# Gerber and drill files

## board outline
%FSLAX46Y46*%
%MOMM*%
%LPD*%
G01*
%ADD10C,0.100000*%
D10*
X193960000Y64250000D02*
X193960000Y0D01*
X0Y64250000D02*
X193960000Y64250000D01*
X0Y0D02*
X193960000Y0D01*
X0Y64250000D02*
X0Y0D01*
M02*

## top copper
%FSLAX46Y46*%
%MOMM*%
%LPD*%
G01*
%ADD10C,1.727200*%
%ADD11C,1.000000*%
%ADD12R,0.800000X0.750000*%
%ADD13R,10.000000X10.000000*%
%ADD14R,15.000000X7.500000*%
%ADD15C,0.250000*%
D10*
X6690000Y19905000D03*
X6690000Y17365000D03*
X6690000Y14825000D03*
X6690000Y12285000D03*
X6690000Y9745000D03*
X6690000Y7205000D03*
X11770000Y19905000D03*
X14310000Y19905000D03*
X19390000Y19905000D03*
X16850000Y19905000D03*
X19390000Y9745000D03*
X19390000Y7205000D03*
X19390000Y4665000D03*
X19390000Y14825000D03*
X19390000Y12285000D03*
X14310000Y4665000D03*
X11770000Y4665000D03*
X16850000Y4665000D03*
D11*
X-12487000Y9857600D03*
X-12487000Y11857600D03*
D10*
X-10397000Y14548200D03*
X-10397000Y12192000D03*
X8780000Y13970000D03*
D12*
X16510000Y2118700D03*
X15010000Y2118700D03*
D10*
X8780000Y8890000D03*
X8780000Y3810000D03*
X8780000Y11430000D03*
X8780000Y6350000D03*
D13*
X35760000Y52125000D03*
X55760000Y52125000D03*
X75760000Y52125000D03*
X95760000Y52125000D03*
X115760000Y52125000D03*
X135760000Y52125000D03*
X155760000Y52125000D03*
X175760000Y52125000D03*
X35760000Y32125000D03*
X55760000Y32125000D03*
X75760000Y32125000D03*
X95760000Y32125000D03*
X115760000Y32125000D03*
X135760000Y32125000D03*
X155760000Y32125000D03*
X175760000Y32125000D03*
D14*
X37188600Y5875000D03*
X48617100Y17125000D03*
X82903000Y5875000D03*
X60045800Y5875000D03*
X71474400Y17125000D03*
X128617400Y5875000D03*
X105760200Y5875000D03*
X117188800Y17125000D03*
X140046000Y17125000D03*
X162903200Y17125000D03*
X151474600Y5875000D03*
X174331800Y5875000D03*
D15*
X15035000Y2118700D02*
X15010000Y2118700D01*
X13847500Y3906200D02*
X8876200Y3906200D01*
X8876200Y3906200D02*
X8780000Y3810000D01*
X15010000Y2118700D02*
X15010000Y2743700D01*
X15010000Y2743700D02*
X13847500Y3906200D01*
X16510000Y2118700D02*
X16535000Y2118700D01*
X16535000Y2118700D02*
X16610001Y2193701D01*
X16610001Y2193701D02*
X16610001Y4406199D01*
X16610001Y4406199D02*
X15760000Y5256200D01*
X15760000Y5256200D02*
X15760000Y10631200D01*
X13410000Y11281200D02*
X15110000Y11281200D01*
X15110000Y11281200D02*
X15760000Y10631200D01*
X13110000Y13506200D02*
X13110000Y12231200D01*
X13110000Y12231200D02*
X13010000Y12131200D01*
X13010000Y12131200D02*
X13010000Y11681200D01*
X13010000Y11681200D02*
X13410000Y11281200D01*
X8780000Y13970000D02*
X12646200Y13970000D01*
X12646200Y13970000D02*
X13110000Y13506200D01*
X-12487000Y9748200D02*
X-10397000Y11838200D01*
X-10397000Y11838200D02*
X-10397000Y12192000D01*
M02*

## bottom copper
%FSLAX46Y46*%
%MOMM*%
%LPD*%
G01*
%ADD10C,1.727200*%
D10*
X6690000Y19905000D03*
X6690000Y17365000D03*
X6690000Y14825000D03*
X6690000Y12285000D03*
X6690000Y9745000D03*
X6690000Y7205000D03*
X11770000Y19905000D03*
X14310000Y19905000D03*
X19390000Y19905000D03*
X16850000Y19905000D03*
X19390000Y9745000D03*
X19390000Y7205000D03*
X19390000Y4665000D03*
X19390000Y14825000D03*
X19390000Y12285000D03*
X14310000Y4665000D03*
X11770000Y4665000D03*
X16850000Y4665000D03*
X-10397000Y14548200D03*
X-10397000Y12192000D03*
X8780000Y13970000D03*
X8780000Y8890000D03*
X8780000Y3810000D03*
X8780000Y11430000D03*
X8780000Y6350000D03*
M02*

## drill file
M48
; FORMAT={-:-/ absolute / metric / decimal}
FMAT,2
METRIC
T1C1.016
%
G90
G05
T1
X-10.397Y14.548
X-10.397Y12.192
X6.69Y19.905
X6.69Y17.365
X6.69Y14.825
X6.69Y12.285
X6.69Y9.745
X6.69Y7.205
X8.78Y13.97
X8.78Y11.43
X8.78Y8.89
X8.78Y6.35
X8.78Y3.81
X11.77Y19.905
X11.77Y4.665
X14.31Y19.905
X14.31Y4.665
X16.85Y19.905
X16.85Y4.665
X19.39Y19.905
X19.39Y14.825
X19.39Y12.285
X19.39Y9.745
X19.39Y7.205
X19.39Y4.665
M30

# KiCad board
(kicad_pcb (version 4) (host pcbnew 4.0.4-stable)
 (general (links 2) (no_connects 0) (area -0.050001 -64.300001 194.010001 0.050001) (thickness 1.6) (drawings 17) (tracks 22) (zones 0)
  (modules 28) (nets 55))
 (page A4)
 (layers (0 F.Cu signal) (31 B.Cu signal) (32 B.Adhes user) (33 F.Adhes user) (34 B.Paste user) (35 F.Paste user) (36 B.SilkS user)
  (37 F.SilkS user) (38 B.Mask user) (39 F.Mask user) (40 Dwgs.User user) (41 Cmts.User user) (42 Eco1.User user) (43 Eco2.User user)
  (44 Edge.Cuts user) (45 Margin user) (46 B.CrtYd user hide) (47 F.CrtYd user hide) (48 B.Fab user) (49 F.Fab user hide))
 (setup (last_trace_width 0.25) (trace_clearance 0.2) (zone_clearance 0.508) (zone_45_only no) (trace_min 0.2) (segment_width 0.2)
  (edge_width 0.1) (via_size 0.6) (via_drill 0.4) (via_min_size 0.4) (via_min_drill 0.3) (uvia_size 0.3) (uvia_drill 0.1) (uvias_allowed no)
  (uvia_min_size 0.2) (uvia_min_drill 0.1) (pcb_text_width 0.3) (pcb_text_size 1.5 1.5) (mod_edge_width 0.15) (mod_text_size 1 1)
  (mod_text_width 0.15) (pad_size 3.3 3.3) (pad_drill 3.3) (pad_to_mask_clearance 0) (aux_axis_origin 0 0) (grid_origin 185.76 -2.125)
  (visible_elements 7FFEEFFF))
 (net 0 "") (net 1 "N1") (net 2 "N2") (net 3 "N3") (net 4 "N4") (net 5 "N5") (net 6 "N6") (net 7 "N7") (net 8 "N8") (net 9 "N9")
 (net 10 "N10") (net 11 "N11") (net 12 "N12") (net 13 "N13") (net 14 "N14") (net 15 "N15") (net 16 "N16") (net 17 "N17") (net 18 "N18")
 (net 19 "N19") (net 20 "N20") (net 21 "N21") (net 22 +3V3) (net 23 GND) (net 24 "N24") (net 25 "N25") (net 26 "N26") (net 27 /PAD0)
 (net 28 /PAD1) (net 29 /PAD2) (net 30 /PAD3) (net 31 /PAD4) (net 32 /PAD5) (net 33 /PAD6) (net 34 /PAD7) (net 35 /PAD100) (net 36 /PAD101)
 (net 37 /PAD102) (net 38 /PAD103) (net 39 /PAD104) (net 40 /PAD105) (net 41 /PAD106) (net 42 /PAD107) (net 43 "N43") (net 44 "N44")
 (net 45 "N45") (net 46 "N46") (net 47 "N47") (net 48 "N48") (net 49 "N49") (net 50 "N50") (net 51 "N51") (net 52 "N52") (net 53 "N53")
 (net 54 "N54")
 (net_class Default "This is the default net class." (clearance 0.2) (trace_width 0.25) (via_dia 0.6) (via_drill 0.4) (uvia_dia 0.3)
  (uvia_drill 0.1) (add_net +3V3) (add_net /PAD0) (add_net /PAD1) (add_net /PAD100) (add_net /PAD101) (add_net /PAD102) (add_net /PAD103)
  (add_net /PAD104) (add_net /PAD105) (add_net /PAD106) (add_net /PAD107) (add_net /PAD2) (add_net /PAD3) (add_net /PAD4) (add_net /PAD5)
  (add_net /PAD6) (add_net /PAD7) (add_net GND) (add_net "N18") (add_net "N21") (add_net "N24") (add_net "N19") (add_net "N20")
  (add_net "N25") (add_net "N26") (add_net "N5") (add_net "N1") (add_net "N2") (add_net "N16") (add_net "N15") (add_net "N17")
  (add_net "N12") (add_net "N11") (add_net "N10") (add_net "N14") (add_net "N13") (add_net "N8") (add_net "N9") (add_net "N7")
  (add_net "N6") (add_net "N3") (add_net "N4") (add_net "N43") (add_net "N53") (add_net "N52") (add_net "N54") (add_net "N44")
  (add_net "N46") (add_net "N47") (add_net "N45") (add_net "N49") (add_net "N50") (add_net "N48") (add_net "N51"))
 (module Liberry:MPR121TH (layer F.Cu) (at 6.69 -19.905)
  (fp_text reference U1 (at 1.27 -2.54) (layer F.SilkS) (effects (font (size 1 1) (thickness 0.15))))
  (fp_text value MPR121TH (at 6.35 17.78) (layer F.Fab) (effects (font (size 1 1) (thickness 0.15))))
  (pad +3V3 thru_hole circle (at 0 0) (size 1.7272 1.7272) (drill 1.016) (layers *.Cu *.Mask))
  (pad GND thru_hole circle (at 0 2.54) (size 1.7272 1.7272) (drill 1.016) (layers *.Cu *.Mask) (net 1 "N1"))
  (pad IRQ thru_hole circle (at 0 5.08) (size 1.7272 1.7272) (drill 1.016) (layers *.Cu *.Mask) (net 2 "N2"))
  (pad SCL thru_hole circle (at 0 7.62) (size 1.7272 1.7272) (drill 1.016) (layers *.Cu *.Mask) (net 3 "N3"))
  (pad SDA thru_hole circle (at 0 10.16) (size 1.7272 1.7272) (drill 1.016) (layers *.Cu *.Mask) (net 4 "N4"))
  (pad ADDR thru_hole circle (at 0 12.7) (size 1.7272 1.7272) (drill 1.016) (layers *.Cu *.Mask) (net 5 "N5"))
  (pad P11 thru_hole circle (at 5.08 0) (size 1.7272 1.7272) (drill 1.016) (layers *.Cu *.Mask) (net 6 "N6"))
  (pad P10 thru_hole circle (at 7.62 0) (size 1.7272 1.7272) (drill 1.016) (layers *.Cu *.Mask) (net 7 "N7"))
  (pad P08 thru_hole circle (at 12.7 0) (size 1.7272 1.7272) (drill 1.016) (layers *.Cu *.Mask) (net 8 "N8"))
  (pad P09 thru_hole circle (at 10.16 0) (size 1.7272 1.7272) (drill 1.016) (layers *.Cu *.Mask) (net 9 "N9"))
  (pad P05 thru_hole circle (at 12.7 10.16) (size 1.7272 1.7272) (drill 1.016) (layers *.Cu *.Mask) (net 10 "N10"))
  (pad P04 thru_hole circle (at 12.7 12.7) (size 1.7272 1.7272) (drill 1.016) (layers *.Cu *.Mask) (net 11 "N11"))
  (pad P03 thru_hole circle (at 12.7 15.24) (size 1.7272 1.7272) (drill 1.016) (layers *.Cu *.Mask) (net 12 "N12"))
  (pad P07 thru_hole circle (at 12.7 5.08) (size 1.7272 1.7272) (drill 1.016) (layers *.Cu *.Mask) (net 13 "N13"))
  (pad P06 thru_hole circle (at 12.7 7.62) (size 1.7272 1.7272) (drill 1.016) (layers *.Cu *.Mask) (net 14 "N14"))
  (pad P01 thru_hole circle (at 7.62 15.24) (size 1.7272 1.7272) (drill 1.016) (layers *.Cu *.Mask) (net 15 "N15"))
  (pad P00 thru_hole circle (at 5.08 15.24) (size 1.7272 1.7272) (drill 1.016) (layers *.Cu *.Mask) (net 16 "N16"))
  (pad P02 thru_hole circle (at 10.16 15.24) (size 1.7272 1.7272) (drill 1.016) (layers *.Cu *.Mask) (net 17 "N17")))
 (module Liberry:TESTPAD (layer F.Cu) (at -12.487 -9.8576)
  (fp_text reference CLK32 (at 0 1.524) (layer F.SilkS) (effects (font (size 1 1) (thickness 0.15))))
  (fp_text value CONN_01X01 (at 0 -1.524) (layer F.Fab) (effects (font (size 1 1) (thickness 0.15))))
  (pad 1 smd circle (at 0 0 270) (size 1 1) (layers F.Cu F.Paste F.Mask) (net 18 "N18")))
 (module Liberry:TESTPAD (layer F.Cu) (at -12.487 -11.8576)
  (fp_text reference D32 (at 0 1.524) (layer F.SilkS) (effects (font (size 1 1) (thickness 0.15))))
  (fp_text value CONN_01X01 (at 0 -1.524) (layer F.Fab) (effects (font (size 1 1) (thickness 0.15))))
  (pad 1 smd circle (at 0 0 270) (size 1 1) (layers F.Cu F.Paste F.Mask) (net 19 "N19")))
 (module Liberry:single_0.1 (layer F.Cu) (at -10.397 -14.5482)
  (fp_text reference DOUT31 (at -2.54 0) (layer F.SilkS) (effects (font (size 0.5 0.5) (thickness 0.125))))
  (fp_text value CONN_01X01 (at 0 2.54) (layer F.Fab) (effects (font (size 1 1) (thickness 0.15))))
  (pad 1 thru_hole circle (at 0 0) (size 1.7272 1.7272) (drill 1.016) (layers *.Cu *.Mask) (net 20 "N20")))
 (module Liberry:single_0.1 (layer F.Cu) (at -10.397 -12.192)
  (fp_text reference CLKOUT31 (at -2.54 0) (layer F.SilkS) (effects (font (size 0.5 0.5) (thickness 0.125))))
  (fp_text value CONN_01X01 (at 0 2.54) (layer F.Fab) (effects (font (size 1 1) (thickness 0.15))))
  (pad 1 thru_hole circle (at 0 0) (size 1.7272 1.7272) (drill 1.016) (layers *.Cu *.Mask) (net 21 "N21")))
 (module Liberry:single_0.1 (layer F.Cu) (at 8.78 -13.97)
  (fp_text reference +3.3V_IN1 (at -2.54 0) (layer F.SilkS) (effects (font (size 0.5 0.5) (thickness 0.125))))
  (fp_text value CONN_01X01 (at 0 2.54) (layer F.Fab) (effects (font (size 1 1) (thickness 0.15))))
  (pad 1 thru_hole circle (at 0 0) (size 1.7272 1.7272) (drill 1.016) (layers *.Cu *.Mask) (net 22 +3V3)))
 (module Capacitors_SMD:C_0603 (layer F.Cu) (at 15.76 -2.1187 180)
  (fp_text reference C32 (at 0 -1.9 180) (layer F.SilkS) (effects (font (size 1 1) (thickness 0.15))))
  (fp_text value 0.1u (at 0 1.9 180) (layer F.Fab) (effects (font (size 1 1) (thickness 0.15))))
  (pad 1 smd rect (at -0.75 0 180) (size 0.8 0.75) (layers F.Cu F.Paste F.Mask) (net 22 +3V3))
  (pad 2 smd rect (at 0.75 0 180) (size 0.8 0.75) (layers F.Cu F.Paste F.Mask) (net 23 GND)))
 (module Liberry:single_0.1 (layer F.Cu) (at 8.78 -8.89)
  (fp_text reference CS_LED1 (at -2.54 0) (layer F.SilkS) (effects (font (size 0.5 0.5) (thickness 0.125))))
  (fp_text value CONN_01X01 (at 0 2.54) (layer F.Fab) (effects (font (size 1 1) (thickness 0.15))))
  (pad 1 thru_hole circle (at 0 0) (size 1.7272 1.7272) (drill 1.016) (layers *.Cu *.Mask) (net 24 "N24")))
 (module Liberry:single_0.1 (layer F.Cu) (at 8.78 -3.81)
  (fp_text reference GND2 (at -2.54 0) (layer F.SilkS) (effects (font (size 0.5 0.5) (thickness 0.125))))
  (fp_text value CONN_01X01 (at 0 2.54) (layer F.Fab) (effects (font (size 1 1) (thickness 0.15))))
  (pad 1 thru_hole circle (at 0 0) (size 1.7272 1.7272) (drill 1.016) (layers *.Cu *.Mask) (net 23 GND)))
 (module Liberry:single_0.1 (layer F.Cu) (at 8.78 -11.43)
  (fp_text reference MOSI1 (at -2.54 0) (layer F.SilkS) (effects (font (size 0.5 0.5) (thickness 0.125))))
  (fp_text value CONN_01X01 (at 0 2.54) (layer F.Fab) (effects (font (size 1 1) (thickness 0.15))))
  (pad 1 thru_hole circle (at 0 0) (size 1.7272 1.7272) (drill 1.016) (layers *.Cu *.Mask) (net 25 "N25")))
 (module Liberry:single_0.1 (layer F.Cu) (at 8.78 -6.35)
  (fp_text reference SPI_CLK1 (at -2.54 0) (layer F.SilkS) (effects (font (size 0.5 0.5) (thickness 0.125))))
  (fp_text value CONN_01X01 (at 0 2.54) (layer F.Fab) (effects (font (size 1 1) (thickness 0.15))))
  (pad 1 thru_hole circle (at 0 0) (size 1.7272 1.7272) (drill 1.016) (layers *.Cu *.Mask) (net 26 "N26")))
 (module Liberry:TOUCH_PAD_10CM (layer F.Cu) (at 35.76 -52.125)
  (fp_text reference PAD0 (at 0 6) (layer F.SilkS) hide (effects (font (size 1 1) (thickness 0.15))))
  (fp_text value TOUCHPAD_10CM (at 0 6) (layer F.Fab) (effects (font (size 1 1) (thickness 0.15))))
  (pad 1 smd rect (at 0 0) (size 10 10) (layers F.Cu) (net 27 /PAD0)))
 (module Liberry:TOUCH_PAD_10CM (layer F.Cu) (at 55.76 -52.125)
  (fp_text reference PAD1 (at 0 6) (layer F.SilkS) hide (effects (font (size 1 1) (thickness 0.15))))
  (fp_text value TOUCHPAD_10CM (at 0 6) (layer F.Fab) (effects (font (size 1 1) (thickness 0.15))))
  (pad 1 smd rect (at 0 0) (size 10 10) (layers F.Cu) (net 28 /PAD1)))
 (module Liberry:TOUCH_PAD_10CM (layer F.Cu) (at 75.76 -52.125)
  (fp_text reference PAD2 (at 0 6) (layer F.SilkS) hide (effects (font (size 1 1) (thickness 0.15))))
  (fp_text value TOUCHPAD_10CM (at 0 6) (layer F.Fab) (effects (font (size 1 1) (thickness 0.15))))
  (pad 1 smd rect (at 0 0) (size 10 10) (layers F.Cu) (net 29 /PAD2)))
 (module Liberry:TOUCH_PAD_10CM (layer F.Cu) (at 95.76 -52.125)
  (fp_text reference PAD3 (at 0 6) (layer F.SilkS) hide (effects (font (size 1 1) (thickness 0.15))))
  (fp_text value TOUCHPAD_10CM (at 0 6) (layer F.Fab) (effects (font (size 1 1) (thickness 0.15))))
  (pad 1 smd rect (at 0 0) (size 10 10) (layers F.Cu) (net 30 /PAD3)))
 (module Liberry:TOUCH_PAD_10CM (layer F.Cu) (at 115.76 -52.125)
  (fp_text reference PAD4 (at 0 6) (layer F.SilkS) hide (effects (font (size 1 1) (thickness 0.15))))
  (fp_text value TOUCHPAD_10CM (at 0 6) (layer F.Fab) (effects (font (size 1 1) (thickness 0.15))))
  (pad 1 smd rect (at 0 0) (size 10 10) (layers F.Cu) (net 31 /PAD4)))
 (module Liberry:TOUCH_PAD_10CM (layer F.Cu) (at 135.76 -52.125)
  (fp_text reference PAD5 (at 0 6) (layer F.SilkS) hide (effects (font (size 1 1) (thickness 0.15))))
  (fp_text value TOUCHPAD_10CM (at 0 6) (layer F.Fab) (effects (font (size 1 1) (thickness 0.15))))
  (pad 1 smd rect (at 0 0) (size 10 10) (layers F.Cu) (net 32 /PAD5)))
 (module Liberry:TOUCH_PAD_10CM (layer F.Cu) (at 155.76 -52.125)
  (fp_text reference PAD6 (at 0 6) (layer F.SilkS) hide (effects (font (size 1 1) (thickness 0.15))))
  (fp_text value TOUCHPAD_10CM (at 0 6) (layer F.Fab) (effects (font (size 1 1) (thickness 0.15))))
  (pad 1 smd rect (at 0 0) (size 10 10) (layers F.Cu) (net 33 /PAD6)))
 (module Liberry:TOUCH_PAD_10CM (layer F.Cu) (at 175.76 -52.125)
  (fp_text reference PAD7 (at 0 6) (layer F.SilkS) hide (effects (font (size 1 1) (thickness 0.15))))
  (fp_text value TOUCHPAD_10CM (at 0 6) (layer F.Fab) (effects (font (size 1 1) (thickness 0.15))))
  (pad 1 smd rect (at 0 0) (size 10 10) (layers F.Cu) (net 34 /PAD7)))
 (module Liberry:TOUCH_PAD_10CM (layer F.Cu) (at 35.76 -32.125)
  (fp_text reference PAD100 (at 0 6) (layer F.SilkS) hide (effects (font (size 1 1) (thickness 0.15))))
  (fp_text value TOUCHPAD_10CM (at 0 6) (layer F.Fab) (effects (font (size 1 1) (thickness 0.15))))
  (pad 1 smd rect (at 0 0) (size 10 10) (layers F.Cu) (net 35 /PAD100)))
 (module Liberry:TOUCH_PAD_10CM (layer F.Cu) (at 55.76 -32.125)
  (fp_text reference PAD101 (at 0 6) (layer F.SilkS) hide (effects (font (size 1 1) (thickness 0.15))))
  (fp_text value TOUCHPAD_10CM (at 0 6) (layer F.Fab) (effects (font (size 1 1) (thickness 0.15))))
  (pad 1 smd rect (at 0 0) (size 10 10) (layers F.Cu) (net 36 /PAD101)))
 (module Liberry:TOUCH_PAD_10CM (layer F.Cu) (at 75.76 -32.125)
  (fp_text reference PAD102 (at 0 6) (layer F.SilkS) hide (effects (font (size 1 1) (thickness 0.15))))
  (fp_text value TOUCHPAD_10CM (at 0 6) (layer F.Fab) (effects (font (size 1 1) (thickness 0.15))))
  (pad 1 smd rect (at 0 0) (size 10 10) (layers F.Cu) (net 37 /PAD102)))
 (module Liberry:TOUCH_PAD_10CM (layer F.Cu) (at 95.76 -32.125)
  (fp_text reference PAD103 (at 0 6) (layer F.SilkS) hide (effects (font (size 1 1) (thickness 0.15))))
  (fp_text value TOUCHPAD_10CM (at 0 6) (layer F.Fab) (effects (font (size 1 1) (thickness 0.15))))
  (pad 1 smd rect (at 0 0) (size 10 10) (layers F.Cu) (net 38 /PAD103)))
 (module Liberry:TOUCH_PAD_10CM (layer F.Cu) (at 115.76 -32.125)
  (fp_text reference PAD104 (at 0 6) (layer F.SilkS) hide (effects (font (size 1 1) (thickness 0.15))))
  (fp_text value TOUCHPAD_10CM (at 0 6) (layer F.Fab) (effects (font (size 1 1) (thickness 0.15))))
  (pad 1 smd rect (at 0 0) (size 10 10) (layers F.Cu) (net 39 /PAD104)))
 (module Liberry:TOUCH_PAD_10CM (layer F.Cu) (at 135.76 -32.125)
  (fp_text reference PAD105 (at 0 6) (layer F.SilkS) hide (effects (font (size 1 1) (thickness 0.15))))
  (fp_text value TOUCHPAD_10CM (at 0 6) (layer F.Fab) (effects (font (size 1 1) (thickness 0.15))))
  (pad 1 smd rect (at 0 0) (size 10 10) (layers F.Cu) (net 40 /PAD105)))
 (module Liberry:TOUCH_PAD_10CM (layer F.Cu) (at 155.76 -32.125)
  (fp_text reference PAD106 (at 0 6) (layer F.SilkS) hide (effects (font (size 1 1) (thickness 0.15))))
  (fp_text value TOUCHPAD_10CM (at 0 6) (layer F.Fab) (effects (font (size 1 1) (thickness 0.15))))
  (pad 1 smd rect (at 0 0) (size 10 10) (layers F.Cu) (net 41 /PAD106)))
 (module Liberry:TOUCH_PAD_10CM (layer F.Cu) (at 175.76 -32.125)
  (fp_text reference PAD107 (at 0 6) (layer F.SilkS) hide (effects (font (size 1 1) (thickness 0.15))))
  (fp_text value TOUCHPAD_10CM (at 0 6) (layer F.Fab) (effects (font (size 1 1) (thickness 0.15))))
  (pad 1 smd rect (at 0 0) (size 10 10) (layers F.Cu) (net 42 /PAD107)))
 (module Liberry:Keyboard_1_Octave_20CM (layer F.Cu) (at 25.76 -2.125)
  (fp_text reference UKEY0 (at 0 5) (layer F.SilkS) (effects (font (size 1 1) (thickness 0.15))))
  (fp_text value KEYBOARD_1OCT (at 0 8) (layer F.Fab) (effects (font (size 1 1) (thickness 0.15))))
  (pad 1 smd rect (at 11.4286 -3.75) (size 15 7.5) (layers F.Cu F.Paste F.Mask) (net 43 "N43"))
  (pad 2 smd rect (at 22.8571 -15) (size 15 7.5) (layers F.Cu F.Paste F.Mask) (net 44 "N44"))
  (pad 5 smd rect (at 57.143 -3.75) (size 15 7.5) (layers F.Cu F.Paste F.Mask) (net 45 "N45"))
  (pad 3 smd rect (at 34.2858 -3.75) (size 15 7.5) (layers F.Cu F.Paste F.Mask) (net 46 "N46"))
  (pad 4 smd rect (at 45.7144 -15) (size 15 7.5) (layers F.Cu F.Paste F.Mask) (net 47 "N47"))
  (pad 8 smd rect (at 102.8574 -3.75) (size 15 7.5) (layers F.Cu F.Paste F.Mask) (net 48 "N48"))
  (pad 6 smd rect (at 80.0002 -3.75) (size 15 7.5) (layers F.Cu F.Paste F.Mask) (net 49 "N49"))
  (pad 7 smd rect (at 91.4288 -15) (size 15 7.5) (layers F.Cu F.Paste F.Mask) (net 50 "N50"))
  (pad 9 smd rect (at 114.286 -15) (size 15 7.5) (layers F.Cu F.Paste F.Mask) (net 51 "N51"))
  (pad 11 smd rect (at 137.1432 -15) (size 15 7.5) (layers F.Cu F.Paste F.Mask) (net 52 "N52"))
  (pad 10 smd rect (at 125.7146 -3.75) (size 15 7.5) (layers F.Cu F.Paste F.Mask) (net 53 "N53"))
  (pad 12 smd rect (at 148.5718 -3.75) (size 15 7.5) (layers F.Cu F.Paste F.Mask) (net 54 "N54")))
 (gr_line (start 193.96 -64.25) (end 193.96 0) (layer Edge.Cuts) (width 0.1))
 (gr_line (start 0 -64.25) (end 193.96 -64.25) (layer Edge.Cuts) (width 0.1))
 (gr_line (start 0 0) (end 193.96 0) (layer Edge.Cuts) (width 0.1))
 (gr_line (start 0 -64.25) (end 0 0) (layer Edge.Cuts) (width 0.1))
 (segment (start 25.76 -2.125) (end 25.76 -32.125) (width 0.25) (layer Dwgs.User) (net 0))
 (segment (start 185.76 -2.125) (end 25.76 -2.125) (width 0.25) (layer Dwgs.User) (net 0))
 (segment (start 15.035 -2.1187) (end 15.01 -2.1187) (width 0.25) (layer F.Cu) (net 23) (status 30))
 (segment (start 13.8475 -3.9062) (end 8.8762 -3.9062) (width 0.25) (layer F.Cu) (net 23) (status 20))
 (segment (start 8.8762 -3.9062) (end 8.78 -3.81) (width 0.25) (layer F.Cu) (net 23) (status 30))
 (segment (start 15.01 -2.1187) (end 15.01 -2.7437) (width 0.25) (layer F.Cu) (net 23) (status 10))
 (segment (start 15.01 -2.7437) (end 13.8475 -3.9062) (width 0.25) (layer F.Cu) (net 23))
 (segment (start 16.51 -2.1187) (end 16.535 -2.1187) (width 0.25) (layer F.Cu) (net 22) (status 30))
 (segment (start 16.535 -2.1187) (end 16.610001 -2.193701) (width 0.25) (layer F.Cu) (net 22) (status 30))
 (segment (start 16.610001 -2.193701) (end 16.610001 -4.406199) (width 0.25) (layer F.Cu) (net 22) (status 10))
 (segment (start 16.610001 -4.406199) (end 15.76 -5.2562) (width 0.25) (layer F.Cu) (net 22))
 (segment (start 15.76 -5.2562) (end 15.76 -10.6312) (width 0.25) (layer F.Cu) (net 22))
 (segment (start 13.41 -11.2812) (end 15.11 -11.2812) (width 0.25) (layer F.Cu) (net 22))
 (segment (start 15.11 -11.2812) (end 15.76 -10.6312) (width 0.25) (layer F.Cu) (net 22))
 (segment (start 13.11 -13.5062) (end 13.11 -12.2312) (width 0.25) (layer F.Cu) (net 22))
 (segment (start 13.11 -12.2312) (end 13.01 -12.1312) (width 0.25) (layer F.Cu) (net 22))
 (segment (start 13.01 -12.1312) (end 13.01 -11.6812) (width 0.25) (layer F.Cu) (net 22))
 (segment (start 13.01 -11.6812) (end 13.41 -11.2812) (width 0.25) (layer F.Cu) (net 22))
 (segment (start 8.78 -13.97) (end 12.6462 -13.97) (width 0.25) (layer F.Cu) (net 22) (status 10))
 (segment (start 12.6462 -13.97) (end 13.11 -13.5062) (width 0.25) (layer F.Cu) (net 22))
 (segment (start -12.487 -9.7482) (end -10.397 -11.8382) (width 0.25) (layer F.Cu) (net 18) (status 30))
 (segment (start -10.397 -11.8382) (end -10.397 -12.192) (width 0.25) (layer F.Cu) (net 21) (status 30)))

